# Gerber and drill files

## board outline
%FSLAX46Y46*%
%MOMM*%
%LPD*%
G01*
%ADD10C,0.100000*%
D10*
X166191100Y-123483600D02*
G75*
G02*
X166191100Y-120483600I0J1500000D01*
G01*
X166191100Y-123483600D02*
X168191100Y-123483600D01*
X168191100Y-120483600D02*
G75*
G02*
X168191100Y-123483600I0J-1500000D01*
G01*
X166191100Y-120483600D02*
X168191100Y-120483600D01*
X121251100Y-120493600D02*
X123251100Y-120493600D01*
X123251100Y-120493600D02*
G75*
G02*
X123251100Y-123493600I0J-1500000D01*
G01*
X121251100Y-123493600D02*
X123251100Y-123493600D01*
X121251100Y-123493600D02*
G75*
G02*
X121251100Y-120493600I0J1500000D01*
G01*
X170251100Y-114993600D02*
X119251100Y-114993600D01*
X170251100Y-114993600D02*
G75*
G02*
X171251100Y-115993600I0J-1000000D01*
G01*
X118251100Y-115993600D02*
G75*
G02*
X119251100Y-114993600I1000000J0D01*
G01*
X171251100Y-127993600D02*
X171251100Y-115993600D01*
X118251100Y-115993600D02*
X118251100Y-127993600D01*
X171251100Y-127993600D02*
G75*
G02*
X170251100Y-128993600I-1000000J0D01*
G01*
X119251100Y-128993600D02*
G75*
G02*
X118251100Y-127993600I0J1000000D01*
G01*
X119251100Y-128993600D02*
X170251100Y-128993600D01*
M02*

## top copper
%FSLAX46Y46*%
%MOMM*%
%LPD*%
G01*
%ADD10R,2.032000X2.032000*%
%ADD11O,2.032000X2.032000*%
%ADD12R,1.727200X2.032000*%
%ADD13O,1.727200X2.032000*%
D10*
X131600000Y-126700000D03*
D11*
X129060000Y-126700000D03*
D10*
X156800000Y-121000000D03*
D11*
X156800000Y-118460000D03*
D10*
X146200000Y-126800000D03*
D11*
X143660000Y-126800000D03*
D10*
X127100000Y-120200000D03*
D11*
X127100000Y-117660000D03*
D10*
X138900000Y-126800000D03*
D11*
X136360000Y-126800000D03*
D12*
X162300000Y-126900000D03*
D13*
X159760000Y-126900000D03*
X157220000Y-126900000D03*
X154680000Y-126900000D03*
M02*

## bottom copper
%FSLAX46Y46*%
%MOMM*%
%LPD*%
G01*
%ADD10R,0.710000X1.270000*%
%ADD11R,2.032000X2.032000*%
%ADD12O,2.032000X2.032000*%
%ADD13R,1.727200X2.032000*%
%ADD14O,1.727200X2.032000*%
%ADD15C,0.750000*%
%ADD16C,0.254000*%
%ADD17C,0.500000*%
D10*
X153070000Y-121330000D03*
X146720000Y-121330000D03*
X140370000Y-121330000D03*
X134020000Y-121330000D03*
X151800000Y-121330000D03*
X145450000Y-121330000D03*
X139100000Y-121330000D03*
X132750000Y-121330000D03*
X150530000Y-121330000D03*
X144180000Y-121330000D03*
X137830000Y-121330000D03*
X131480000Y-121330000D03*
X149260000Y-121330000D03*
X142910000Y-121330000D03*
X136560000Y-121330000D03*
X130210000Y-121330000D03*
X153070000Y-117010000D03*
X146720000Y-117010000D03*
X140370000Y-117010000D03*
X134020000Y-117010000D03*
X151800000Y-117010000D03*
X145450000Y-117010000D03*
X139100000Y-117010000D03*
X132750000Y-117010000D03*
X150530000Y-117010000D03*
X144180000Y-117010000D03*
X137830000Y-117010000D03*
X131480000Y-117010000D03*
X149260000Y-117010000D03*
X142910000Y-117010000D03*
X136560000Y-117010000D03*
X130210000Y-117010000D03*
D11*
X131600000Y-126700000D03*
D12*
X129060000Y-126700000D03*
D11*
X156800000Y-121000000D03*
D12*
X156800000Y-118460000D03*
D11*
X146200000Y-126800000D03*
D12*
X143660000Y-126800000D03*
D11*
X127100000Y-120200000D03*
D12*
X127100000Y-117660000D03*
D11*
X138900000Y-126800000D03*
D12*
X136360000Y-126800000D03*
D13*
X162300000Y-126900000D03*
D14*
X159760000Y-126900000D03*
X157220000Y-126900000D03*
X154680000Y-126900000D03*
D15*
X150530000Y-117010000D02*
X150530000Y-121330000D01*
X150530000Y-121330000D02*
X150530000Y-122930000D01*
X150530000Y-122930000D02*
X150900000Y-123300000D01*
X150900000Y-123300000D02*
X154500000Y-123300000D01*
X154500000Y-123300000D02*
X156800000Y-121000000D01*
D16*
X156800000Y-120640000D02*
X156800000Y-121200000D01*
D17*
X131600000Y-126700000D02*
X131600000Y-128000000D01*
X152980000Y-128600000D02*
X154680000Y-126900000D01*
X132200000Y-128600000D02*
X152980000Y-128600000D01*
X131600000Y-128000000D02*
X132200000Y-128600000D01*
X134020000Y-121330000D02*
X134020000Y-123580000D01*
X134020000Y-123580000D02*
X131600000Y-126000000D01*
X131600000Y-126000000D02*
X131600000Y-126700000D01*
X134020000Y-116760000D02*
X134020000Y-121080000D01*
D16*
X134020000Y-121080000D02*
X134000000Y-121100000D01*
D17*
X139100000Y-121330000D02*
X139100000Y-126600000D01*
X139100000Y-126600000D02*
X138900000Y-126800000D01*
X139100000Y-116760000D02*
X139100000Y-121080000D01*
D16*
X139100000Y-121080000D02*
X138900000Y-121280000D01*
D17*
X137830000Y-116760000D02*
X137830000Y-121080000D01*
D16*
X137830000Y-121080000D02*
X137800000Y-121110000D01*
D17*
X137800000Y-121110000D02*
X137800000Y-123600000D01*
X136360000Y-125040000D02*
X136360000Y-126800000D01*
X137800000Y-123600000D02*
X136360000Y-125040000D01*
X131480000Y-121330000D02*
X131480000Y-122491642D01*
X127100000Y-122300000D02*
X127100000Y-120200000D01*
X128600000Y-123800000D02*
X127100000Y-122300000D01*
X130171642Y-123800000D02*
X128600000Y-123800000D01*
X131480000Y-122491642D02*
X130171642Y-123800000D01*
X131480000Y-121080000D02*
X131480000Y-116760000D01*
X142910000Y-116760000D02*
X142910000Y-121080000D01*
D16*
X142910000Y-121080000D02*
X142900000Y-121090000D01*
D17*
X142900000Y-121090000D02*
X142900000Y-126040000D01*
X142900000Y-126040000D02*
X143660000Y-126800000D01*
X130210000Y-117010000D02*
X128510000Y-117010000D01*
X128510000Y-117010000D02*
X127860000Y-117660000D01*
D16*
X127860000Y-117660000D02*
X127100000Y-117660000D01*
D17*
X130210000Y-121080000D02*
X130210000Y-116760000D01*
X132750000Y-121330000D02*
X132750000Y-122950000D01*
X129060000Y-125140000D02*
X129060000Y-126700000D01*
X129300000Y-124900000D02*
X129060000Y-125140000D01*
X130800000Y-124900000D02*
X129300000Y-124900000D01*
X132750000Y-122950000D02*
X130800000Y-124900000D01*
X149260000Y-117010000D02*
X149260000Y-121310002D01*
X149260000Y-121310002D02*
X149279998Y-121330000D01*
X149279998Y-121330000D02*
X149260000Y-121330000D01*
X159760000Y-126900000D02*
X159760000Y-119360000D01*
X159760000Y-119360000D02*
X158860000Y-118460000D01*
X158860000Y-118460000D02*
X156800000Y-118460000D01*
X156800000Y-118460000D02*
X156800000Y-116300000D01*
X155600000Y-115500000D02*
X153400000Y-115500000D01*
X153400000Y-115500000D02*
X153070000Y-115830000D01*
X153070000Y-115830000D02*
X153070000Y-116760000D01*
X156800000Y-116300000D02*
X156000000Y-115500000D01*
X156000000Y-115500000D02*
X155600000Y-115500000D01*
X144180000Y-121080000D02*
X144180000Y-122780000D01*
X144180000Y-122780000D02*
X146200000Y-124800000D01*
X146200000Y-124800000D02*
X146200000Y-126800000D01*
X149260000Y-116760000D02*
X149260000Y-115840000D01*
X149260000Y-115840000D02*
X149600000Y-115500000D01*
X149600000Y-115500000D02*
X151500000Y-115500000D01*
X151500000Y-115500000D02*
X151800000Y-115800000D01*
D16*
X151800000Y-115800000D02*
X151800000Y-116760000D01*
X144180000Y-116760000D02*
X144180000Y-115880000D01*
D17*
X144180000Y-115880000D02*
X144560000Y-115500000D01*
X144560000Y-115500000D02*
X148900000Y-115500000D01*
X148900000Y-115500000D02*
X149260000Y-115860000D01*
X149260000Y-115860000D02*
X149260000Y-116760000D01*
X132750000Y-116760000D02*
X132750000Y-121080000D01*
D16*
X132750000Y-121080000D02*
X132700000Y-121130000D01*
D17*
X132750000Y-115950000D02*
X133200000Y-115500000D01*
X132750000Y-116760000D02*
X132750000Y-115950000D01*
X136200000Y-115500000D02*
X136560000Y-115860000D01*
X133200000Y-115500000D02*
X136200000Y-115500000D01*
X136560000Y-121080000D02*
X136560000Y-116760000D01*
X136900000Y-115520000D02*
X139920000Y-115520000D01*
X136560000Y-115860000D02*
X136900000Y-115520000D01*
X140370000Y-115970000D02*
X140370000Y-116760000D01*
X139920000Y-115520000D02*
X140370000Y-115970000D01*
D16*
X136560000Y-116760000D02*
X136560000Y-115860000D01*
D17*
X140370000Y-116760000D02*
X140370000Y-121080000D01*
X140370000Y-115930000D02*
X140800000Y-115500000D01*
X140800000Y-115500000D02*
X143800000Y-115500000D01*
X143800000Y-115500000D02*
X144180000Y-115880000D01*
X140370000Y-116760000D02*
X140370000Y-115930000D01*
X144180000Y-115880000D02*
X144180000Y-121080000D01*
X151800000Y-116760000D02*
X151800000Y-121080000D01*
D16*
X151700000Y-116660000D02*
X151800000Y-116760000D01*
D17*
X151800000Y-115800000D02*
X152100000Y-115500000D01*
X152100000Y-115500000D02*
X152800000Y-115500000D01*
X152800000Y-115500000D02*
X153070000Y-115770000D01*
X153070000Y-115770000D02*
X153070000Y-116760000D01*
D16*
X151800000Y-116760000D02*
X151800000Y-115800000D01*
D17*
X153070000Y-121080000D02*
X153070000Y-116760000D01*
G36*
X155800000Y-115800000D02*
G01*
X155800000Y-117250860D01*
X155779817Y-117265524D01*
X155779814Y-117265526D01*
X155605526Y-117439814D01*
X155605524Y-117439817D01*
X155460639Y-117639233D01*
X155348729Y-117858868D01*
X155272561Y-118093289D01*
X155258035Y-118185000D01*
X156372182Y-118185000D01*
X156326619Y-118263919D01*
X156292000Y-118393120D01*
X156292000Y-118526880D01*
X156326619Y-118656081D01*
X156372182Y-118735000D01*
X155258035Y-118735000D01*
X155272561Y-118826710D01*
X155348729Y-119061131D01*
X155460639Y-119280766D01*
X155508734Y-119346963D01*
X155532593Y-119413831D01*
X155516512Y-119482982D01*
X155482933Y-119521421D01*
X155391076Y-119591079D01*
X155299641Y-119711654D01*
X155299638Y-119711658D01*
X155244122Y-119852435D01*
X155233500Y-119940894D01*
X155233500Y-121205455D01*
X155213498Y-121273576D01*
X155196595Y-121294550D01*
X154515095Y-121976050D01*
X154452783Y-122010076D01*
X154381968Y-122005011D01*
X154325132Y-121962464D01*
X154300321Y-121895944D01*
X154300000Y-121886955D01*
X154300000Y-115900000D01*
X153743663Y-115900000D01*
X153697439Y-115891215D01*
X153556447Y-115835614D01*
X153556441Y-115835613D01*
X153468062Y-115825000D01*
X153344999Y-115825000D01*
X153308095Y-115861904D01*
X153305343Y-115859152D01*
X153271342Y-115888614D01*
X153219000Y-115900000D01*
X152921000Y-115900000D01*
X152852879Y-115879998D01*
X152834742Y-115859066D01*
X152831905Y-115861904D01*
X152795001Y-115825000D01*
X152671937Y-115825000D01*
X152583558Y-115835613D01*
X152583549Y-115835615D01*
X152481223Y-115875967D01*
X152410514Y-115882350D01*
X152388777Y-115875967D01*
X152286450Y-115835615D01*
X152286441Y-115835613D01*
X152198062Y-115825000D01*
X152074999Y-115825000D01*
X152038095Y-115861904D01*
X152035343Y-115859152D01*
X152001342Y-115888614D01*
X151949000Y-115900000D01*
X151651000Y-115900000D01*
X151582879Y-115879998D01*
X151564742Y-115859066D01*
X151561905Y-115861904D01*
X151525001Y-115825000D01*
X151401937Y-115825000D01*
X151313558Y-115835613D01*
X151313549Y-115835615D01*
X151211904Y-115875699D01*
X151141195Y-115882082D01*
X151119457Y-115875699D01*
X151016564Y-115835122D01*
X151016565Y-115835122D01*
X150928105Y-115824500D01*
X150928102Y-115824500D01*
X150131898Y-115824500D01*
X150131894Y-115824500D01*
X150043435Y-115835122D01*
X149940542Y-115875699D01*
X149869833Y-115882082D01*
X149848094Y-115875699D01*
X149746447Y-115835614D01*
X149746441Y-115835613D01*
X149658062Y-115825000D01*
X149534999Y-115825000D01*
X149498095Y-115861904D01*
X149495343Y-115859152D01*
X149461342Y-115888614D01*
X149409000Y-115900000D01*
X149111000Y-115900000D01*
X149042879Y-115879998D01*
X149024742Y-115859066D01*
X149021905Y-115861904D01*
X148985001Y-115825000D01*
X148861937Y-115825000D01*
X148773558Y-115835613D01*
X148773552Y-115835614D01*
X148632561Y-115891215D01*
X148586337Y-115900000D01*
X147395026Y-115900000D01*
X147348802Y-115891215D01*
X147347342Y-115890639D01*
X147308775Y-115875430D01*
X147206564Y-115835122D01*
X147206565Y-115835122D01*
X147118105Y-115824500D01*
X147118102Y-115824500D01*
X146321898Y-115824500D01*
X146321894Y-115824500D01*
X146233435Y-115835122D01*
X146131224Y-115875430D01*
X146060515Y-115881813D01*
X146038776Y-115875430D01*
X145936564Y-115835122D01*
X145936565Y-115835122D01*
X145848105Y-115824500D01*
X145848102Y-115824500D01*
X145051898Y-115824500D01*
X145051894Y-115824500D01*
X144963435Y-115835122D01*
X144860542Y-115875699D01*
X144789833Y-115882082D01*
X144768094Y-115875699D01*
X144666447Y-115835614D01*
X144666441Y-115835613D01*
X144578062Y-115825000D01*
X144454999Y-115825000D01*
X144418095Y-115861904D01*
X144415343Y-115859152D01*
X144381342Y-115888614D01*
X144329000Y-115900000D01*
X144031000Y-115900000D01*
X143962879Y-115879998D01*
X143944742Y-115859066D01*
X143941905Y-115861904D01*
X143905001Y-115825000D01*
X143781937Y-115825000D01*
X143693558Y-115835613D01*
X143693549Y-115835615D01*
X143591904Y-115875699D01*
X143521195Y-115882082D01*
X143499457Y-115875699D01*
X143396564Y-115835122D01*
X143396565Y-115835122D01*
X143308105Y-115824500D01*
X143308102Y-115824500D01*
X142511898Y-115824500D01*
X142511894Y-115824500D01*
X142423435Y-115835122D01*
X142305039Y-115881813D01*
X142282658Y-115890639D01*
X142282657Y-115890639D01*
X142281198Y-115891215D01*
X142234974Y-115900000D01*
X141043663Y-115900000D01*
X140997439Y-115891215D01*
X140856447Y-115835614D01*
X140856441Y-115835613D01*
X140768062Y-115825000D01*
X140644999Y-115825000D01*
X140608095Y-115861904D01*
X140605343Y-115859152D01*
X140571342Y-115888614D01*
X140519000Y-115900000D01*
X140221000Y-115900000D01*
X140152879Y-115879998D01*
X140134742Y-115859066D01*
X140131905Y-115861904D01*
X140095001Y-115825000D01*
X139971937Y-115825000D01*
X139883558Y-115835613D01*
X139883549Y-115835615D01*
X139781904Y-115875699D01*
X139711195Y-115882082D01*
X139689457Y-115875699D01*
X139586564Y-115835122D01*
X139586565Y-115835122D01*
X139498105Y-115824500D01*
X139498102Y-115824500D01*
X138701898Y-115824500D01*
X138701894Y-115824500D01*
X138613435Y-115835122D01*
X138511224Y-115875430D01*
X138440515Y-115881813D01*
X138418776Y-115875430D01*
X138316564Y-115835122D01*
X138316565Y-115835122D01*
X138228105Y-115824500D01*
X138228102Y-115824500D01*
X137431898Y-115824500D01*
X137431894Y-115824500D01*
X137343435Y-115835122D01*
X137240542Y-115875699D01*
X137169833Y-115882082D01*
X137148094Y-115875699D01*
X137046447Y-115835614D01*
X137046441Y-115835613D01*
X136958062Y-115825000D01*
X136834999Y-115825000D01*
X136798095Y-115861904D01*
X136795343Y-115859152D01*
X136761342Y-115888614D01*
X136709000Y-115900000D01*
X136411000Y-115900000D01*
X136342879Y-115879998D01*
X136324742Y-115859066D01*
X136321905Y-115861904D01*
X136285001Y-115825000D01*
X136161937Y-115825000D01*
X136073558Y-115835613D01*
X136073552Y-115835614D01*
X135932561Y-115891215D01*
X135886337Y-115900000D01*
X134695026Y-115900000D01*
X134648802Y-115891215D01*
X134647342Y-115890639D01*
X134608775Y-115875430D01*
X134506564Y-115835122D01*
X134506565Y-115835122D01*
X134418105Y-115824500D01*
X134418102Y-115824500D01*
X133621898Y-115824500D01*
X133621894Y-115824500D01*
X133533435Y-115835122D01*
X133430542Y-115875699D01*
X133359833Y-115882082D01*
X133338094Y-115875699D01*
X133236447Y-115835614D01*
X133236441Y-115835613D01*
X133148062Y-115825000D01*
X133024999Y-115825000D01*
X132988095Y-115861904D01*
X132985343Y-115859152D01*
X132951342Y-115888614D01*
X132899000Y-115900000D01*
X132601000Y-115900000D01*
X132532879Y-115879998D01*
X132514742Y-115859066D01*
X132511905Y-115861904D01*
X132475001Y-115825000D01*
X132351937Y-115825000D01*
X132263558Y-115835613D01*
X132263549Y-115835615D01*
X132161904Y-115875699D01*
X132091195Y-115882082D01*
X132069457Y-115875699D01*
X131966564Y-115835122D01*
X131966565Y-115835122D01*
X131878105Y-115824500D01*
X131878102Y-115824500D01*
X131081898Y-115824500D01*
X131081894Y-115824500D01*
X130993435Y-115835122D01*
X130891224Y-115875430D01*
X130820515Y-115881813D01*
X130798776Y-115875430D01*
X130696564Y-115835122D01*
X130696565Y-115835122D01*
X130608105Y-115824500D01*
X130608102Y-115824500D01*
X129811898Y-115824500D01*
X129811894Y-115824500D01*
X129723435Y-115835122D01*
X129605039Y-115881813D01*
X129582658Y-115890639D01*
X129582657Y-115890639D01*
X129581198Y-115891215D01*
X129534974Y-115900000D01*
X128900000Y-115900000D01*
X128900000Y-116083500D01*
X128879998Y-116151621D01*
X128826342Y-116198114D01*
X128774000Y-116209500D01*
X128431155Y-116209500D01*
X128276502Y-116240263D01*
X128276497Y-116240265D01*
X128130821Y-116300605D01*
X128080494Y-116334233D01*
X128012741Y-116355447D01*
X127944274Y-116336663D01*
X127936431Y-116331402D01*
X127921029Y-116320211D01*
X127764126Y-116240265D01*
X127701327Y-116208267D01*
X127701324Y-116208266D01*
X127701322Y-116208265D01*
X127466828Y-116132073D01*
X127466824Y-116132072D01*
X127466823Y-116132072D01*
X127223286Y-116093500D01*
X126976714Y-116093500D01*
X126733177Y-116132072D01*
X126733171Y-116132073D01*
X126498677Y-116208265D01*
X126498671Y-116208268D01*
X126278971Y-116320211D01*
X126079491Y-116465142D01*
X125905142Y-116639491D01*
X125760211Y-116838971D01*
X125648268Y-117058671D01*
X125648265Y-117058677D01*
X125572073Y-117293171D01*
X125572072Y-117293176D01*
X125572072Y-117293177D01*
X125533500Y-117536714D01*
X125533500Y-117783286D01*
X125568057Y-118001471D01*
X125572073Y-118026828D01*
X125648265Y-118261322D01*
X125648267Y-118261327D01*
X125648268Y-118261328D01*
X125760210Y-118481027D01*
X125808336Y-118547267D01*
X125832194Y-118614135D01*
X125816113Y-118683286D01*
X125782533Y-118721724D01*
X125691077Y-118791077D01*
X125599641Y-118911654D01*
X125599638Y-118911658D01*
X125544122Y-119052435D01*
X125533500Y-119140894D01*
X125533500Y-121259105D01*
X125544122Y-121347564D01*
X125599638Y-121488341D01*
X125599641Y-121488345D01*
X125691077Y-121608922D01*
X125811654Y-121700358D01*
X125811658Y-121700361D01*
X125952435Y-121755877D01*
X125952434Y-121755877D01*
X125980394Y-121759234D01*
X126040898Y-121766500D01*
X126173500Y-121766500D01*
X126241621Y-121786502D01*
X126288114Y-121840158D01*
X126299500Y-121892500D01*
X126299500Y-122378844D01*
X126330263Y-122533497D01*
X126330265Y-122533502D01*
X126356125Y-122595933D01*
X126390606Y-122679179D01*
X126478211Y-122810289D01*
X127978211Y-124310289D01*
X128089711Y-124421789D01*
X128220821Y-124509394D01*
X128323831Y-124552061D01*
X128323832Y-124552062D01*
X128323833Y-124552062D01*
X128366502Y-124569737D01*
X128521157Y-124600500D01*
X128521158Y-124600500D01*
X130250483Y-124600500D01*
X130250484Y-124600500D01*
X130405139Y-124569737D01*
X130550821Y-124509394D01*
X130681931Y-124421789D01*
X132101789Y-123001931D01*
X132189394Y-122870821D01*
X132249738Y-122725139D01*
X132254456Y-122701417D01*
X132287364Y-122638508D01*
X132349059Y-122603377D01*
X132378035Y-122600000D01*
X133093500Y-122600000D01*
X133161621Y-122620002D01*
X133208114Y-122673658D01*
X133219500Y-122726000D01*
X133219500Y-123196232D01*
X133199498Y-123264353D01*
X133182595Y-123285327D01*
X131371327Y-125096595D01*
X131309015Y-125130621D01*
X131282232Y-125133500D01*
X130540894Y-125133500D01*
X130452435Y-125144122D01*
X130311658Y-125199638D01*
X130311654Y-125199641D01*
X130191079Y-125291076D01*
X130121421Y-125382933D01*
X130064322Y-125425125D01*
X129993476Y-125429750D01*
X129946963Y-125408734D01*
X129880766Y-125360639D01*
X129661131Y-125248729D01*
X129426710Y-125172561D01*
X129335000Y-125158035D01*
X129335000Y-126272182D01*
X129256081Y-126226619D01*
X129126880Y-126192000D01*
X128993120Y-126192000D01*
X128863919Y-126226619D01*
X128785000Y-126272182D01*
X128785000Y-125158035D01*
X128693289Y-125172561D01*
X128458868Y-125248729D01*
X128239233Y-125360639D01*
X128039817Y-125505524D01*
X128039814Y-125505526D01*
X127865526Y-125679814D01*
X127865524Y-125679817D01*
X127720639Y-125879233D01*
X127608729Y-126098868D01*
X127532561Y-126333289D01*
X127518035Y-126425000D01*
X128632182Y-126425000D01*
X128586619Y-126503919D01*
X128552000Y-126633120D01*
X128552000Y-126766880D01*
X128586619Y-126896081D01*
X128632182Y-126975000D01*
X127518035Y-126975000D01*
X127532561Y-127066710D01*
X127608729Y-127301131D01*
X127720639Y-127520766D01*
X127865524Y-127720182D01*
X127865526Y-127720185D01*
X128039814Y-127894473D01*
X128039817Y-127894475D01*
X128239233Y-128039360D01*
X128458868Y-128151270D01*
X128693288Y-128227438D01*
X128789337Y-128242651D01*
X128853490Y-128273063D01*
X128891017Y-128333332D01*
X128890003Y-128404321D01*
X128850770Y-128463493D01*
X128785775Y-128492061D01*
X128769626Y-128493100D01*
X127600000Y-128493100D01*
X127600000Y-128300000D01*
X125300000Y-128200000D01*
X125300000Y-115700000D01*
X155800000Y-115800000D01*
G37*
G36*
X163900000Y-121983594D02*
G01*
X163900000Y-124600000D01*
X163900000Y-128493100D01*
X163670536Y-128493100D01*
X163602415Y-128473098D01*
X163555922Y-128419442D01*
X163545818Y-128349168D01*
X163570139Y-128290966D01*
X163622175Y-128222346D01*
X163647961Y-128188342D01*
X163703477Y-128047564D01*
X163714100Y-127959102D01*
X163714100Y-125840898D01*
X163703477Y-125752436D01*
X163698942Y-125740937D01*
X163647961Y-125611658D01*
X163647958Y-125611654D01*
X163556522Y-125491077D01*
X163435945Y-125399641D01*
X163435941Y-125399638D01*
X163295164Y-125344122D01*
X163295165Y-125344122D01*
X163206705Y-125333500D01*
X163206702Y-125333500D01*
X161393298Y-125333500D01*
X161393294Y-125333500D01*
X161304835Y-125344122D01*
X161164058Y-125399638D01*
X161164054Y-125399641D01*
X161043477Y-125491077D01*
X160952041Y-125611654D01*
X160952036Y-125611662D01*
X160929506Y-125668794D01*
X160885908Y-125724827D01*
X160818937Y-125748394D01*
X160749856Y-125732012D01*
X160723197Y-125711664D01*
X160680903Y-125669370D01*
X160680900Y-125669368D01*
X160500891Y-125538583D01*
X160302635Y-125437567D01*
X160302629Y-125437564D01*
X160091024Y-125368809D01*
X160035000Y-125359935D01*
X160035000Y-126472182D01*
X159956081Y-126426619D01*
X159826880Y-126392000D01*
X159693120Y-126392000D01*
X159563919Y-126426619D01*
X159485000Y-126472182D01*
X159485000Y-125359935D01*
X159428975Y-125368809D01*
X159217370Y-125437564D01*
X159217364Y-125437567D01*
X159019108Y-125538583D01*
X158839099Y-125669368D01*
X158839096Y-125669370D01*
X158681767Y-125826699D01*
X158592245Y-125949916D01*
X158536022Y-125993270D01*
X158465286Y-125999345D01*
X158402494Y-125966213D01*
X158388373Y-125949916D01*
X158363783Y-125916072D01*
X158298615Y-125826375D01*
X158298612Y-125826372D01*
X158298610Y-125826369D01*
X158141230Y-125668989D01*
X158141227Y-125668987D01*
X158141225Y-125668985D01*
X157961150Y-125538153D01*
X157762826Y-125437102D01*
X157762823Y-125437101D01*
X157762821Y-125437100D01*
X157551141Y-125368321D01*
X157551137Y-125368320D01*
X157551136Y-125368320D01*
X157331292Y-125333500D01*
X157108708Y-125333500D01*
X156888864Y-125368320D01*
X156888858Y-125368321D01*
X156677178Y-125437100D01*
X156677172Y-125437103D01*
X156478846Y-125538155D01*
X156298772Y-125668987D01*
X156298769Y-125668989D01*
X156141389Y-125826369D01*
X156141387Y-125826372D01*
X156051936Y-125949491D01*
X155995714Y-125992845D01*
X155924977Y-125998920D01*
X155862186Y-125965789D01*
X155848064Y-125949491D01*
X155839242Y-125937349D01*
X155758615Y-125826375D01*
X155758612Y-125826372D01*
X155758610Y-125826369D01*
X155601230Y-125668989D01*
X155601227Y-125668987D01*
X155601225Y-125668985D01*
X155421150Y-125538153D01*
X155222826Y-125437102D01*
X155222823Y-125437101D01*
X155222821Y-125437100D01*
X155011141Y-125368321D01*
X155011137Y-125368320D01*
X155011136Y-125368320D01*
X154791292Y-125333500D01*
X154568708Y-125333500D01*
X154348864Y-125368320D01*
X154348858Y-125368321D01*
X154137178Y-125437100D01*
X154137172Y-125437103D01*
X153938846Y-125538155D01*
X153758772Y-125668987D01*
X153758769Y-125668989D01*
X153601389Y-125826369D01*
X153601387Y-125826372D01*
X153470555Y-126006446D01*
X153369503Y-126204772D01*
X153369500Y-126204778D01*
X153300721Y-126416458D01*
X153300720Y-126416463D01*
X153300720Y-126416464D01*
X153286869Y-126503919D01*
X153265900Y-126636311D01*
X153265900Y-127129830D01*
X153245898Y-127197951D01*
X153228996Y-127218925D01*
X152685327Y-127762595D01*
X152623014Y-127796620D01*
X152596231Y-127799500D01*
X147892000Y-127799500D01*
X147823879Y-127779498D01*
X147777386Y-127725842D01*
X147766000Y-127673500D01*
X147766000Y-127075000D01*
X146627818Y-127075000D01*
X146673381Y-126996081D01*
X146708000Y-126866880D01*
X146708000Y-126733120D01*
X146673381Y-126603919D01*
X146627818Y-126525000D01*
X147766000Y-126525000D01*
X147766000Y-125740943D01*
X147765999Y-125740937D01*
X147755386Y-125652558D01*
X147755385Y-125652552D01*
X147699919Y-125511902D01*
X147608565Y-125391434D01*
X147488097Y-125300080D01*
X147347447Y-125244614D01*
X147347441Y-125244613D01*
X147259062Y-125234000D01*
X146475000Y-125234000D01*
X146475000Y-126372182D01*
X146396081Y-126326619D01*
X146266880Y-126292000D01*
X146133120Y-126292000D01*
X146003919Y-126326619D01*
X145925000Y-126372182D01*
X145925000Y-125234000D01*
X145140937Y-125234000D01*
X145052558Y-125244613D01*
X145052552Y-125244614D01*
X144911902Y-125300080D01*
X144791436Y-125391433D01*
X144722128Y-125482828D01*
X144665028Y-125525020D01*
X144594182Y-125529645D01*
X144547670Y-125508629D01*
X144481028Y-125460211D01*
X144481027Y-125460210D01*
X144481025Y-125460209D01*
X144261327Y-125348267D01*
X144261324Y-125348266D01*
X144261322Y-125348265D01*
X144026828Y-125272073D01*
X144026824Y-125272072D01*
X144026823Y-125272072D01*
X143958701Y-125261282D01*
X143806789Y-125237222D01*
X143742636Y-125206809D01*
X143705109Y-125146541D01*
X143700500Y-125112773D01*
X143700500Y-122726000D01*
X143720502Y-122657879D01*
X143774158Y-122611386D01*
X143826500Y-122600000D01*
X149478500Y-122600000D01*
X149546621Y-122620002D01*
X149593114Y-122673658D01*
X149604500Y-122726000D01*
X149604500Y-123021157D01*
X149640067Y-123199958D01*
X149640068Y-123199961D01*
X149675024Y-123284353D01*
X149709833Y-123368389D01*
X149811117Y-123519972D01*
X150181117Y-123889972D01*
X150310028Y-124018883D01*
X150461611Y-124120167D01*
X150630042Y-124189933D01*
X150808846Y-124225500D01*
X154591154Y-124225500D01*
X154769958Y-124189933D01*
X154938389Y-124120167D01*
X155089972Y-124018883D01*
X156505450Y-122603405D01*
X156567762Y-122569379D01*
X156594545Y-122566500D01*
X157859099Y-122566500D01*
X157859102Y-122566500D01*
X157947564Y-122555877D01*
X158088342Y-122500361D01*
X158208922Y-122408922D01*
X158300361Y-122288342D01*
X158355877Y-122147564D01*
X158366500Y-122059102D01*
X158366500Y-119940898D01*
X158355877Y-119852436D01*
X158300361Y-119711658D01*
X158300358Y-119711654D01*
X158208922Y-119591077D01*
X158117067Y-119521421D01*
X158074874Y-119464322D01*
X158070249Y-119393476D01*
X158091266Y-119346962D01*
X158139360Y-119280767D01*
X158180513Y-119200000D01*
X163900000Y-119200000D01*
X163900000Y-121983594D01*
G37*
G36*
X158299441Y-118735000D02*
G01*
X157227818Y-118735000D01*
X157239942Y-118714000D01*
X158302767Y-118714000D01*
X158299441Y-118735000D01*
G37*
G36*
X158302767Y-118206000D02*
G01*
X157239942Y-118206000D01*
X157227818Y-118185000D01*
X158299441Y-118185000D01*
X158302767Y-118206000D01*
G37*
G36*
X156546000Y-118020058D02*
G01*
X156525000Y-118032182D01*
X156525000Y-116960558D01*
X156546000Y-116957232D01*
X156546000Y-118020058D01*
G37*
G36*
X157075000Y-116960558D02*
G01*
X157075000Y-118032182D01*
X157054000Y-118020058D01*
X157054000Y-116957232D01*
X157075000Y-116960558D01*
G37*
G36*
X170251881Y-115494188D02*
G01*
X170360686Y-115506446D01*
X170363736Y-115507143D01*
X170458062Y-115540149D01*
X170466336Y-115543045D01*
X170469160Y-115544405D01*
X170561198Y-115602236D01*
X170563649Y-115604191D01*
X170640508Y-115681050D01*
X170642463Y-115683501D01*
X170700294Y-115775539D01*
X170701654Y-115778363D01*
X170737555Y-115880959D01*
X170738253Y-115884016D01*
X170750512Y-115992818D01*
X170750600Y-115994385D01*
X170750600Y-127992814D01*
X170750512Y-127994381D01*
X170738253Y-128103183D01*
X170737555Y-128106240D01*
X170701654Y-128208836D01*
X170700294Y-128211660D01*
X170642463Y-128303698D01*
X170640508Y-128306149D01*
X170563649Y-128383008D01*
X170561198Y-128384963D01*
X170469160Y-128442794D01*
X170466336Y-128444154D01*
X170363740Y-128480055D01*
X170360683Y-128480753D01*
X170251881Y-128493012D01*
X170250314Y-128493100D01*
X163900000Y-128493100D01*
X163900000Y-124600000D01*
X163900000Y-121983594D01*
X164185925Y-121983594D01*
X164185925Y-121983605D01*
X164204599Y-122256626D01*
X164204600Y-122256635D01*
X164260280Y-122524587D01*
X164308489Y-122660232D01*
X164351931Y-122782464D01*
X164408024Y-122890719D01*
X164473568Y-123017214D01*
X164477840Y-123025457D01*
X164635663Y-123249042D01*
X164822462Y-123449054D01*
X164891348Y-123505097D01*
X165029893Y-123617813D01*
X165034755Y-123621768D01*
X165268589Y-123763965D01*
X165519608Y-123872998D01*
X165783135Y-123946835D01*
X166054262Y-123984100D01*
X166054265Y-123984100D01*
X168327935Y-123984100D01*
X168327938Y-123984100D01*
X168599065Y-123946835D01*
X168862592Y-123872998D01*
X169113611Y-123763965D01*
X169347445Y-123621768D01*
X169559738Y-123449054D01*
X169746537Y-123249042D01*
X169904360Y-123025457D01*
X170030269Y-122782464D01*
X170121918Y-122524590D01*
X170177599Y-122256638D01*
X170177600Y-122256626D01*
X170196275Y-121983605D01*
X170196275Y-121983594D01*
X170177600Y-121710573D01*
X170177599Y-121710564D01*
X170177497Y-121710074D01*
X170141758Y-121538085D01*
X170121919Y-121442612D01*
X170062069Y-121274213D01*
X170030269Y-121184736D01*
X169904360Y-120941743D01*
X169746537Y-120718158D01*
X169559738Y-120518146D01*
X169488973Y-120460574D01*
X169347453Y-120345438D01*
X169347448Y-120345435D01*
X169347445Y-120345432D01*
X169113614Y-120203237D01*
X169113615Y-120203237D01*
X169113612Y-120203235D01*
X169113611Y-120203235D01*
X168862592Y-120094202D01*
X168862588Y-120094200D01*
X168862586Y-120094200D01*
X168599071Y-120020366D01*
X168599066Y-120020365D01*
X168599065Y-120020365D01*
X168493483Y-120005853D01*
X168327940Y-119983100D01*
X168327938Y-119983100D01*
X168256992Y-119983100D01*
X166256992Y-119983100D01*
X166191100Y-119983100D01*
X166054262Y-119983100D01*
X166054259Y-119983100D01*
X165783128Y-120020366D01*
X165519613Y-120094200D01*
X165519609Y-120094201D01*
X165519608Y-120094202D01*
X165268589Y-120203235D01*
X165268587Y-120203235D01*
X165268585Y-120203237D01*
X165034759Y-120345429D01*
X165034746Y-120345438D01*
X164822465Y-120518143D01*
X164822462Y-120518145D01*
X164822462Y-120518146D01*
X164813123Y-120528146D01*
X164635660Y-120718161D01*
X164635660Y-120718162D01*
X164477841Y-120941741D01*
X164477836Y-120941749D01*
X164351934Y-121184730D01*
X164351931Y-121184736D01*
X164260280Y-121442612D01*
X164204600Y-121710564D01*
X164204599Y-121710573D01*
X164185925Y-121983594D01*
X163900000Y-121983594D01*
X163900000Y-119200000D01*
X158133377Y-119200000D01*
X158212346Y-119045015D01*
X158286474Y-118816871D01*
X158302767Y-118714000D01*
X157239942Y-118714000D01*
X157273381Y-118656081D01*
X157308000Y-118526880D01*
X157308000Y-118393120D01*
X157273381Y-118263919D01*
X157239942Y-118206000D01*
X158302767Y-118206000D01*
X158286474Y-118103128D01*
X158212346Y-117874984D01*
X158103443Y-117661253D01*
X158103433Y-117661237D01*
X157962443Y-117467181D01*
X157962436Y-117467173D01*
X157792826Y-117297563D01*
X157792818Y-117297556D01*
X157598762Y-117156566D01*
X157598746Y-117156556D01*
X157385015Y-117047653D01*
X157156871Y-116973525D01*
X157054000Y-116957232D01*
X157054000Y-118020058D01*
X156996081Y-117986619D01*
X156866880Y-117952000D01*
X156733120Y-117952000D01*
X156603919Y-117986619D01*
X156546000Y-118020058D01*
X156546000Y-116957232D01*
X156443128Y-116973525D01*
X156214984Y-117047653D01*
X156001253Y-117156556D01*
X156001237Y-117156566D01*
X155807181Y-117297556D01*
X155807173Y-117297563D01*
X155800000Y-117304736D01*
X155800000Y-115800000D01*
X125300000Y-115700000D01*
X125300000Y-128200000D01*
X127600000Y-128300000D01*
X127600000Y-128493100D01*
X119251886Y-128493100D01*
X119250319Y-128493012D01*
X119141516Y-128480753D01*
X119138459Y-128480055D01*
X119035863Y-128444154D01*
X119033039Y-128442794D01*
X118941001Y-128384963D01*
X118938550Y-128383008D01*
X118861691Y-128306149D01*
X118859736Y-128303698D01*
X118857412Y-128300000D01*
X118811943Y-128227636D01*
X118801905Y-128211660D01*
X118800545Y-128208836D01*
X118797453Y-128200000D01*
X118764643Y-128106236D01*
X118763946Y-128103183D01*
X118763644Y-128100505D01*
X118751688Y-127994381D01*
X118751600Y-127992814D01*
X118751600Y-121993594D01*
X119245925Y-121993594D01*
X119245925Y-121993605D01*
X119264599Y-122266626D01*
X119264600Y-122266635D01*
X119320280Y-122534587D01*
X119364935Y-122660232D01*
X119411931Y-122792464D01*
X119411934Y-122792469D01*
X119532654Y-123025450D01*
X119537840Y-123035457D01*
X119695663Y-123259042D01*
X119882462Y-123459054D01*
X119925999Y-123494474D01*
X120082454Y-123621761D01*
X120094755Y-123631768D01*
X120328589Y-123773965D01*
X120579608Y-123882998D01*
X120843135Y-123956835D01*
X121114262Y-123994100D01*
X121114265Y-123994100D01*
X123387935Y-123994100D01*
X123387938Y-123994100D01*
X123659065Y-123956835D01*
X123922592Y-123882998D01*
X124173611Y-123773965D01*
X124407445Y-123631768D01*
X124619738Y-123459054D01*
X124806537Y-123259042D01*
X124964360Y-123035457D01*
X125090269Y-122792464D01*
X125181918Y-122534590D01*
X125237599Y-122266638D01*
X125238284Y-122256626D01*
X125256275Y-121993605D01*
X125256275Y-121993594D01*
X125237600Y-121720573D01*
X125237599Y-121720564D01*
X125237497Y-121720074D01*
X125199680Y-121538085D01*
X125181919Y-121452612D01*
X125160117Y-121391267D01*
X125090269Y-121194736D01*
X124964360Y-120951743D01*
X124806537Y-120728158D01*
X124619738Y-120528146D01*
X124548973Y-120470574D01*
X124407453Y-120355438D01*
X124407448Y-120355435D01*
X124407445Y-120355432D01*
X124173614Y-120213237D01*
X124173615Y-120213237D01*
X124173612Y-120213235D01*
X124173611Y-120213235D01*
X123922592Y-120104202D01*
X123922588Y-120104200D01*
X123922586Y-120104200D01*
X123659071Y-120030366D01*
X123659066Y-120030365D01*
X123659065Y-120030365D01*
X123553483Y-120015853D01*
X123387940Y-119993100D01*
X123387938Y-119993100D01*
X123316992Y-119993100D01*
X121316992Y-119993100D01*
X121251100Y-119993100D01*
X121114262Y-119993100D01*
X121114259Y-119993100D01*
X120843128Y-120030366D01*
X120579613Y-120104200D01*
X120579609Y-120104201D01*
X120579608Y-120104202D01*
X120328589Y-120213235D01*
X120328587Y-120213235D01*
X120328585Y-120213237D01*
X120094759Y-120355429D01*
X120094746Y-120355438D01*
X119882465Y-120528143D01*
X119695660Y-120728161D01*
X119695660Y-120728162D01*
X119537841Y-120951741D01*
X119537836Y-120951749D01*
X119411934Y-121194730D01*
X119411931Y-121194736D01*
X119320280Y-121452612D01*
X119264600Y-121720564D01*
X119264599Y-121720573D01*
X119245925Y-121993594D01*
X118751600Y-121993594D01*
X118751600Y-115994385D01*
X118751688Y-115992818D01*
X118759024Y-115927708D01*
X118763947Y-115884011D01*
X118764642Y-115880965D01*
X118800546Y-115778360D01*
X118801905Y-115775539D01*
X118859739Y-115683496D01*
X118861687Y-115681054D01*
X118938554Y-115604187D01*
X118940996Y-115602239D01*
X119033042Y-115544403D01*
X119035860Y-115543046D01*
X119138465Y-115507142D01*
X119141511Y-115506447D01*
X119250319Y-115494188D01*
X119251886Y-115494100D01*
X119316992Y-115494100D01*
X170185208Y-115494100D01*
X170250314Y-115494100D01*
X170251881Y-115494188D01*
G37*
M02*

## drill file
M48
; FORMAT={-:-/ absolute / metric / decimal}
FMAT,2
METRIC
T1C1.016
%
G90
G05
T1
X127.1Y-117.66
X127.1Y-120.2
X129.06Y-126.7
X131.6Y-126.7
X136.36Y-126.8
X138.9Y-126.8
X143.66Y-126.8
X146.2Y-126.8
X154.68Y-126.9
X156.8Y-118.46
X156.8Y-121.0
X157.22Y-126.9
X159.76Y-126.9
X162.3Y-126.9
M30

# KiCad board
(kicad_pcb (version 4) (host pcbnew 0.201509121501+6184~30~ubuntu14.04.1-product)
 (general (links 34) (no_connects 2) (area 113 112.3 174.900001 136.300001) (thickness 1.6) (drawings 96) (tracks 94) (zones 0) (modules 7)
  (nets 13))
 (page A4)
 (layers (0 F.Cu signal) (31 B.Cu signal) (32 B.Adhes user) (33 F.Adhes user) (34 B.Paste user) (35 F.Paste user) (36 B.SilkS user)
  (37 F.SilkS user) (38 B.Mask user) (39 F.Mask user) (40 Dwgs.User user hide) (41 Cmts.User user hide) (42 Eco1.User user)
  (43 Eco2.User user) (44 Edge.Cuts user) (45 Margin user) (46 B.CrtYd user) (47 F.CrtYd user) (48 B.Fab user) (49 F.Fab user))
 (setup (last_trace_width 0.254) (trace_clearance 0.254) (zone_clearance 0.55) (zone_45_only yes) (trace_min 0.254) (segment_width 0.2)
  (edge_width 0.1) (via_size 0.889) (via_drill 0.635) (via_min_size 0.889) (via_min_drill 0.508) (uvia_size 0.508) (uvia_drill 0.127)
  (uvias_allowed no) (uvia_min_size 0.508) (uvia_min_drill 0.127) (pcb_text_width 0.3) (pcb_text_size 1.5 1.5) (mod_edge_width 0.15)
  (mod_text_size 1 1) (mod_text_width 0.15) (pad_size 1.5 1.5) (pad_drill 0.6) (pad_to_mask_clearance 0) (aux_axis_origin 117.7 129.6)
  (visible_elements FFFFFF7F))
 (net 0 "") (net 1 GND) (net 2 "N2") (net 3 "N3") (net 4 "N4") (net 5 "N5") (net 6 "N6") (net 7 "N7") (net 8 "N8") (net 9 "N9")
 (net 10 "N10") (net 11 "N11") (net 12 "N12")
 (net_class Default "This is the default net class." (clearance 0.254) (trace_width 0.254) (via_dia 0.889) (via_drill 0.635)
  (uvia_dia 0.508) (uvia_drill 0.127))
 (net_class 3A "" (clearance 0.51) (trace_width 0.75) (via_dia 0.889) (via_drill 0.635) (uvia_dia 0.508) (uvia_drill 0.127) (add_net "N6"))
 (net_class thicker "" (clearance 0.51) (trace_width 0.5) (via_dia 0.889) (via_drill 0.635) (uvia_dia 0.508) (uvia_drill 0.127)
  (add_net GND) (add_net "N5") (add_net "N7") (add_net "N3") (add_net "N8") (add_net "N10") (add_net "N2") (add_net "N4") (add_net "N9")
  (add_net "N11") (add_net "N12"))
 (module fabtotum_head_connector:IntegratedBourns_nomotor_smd (layer B.Cu) (at 153 121.35 90)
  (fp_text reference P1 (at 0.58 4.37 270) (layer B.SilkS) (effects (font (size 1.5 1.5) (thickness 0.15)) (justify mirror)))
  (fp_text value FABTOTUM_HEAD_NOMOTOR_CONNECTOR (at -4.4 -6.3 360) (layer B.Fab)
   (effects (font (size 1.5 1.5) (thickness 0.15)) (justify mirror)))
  (pad 1 smd rect (at 0.02 0.07 90) (size 1.27 0.71) (layers B.Cu B.Paste B.Mask) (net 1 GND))
  (pad 5 smd rect (at 0.02 -6.28 90) (size 1.27 0.71) (layers B.Cu B.Paste B.Mask) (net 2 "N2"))
  (pad 9 smd rect (at 0.02 -12.63 90) (size 1.27 0.71) (layers B.Cu B.Paste B.Mask) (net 1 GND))
  (pad 13 smd rect (at 0.02 -18.98 90) (size 1.27 0.71) (layers B.Cu B.Paste B.Mask) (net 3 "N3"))
  (pad 2 smd rect (at 0.02 -1.2 90) (size 1.27 0.71) (layers B.Cu B.Paste B.Mask) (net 1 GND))
  (pad 6 smd rect (at 0.02 -7.55 90) (size 1.27 0.71) (layers B.Cu B.Paste B.Mask) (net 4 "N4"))
  (pad 10 smd rect (at 0.02 -13.9 90) (size 1.27 0.71) (layers B.Cu B.Paste B.Mask) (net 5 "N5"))
  (pad 14 smd rect (at 0.02 -20.25 90) (size 1.27 0.71) (layers B.Cu B.Paste B.Mask) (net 1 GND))
  (pad 3 smd rect (at 0.02 -2.47 90) (size 1.27 0.71) (layers B.Cu B.Paste B.Mask) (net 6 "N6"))
  (pad 7 smd rect (at 0.02 -8.82 90) (size 1.27 0.71) (layers B.Cu B.Paste B.Mask) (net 1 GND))
  (pad 11 smd rect (at 0.02 -15.17 90) (size 1.27 0.71) (layers B.Cu B.Paste B.Mask) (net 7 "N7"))
  (pad 15 smd rect (at 0.02 -21.52 90) (size 1.27 0.71) (layers B.Cu B.Paste B.Mask) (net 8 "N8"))
  (pad 4 smd rect (at 0.02 -3.74 90) (size 1.27 0.71) (layers B.Cu B.Paste B.Mask) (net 1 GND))
  (pad 8 smd rect (at 0.02 -10.09 90) (size 1.27 0.71) (layers B.Cu B.Paste B.Mask) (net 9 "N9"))
  (pad 12 smd rect (at 0.02 -16.44 90) (size 1.27 0.71) (layers B.Cu B.Paste B.Mask) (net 1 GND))
  (pad 16 smd rect (at 0.02 -22.79 90) (size 1.27 0.71) (layers B.Cu B.Paste B.Mask) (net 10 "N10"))
  (pad 1 smd rect (at 4.34 0.07 90) (size 1.27 0.71) (layers B.Cu B.Paste B.Mask) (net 1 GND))
  (pad 5 smd rect (at 4.34 -6.28 90) (size 1.27 0.71) (layers B.Cu B.Paste B.Mask) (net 2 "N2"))
  (pad 9 smd rect (at 4.34 -12.63 90) (size 1.27 0.71) (layers B.Cu B.Paste B.Mask) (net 1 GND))
  (pad 13 smd rect (at 4.34 -18.98 90) (size 1.27 0.71) (layers B.Cu B.Paste B.Mask) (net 3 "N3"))
  (pad 2 smd rect (at 4.34 -1.2 90) (size 1.27 0.71) (layers B.Cu B.Paste B.Mask) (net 1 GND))
  (pad 6 smd rect (at 4.34 -7.55 90) (size 1.27 0.71) (layers B.Cu B.Paste B.Mask) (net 4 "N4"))
  (pad 10 smd rect (at 4.34 -13.9 90) (size 1.27 0.71) (layers B.Cu B.Paste B.Mask) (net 5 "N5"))
  (pad 14 smd rect (at 4.34 -20.25 90) (size 1.27 0.71) (layers B.Cu B.Paste B.Mask) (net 1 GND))
  (pad 3 smd rect (at 4.34 -2.47 90) (size 1.27 0.71) (layers B.Cu B.Paste B.Mask) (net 6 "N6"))
  (pad 7 smd rect (at 4.34 -8.82 90) (size 1.27 0.71) (layers B.Cu B.Paste B.Mask) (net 1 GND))
  (pad 11 smd rect (at 4.34 -15.17 90) (size 1.27 0.71) (layers B.Cu B.Paste B.Mask) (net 7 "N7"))
  (pad 15 smd rect (at 4.34 -21.52 90) (size 1.27 0.71) (layers B.Cu B.Paste B.Mask) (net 8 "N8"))
  (pad 4 smd rect (at 4.34 -3.74 90) (size 1.27 0.71) (layers B.Cu B.Paste B.Mask) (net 1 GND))
  (pad 8 smd rect (at 4.34 -10.09 90) (size 1.27 0.71) (layers B.Cu B.Paste B.Mask) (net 9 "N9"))
  (pad 12 smd rect (at 4.34 -16.44 90) (size 1.27 0.71) (layers B.Cu B.Paste B.Mask) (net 1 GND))
  (pad 16 smd rect (at 4.34 -22.79 90) (size 1.27 0.71) (layers B.Cu B.Paste B.Mask) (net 10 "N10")))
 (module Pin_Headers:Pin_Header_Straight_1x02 (layer F.Cu) (at 131.6 126.7 270)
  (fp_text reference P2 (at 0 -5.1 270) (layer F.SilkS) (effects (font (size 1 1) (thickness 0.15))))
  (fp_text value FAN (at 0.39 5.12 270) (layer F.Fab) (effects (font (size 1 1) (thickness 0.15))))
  (pad 1 thru_hole rect (at 0 0 270) (size 2.032 2.032) (drill 1.016) (layers *.Cu *.Mask F.SilkS) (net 3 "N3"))
  (pad 2 thru_hole oval (at 0 2.54 270) (size 2.032 2.032) (drill 1.016) (layers *.Cu *.Mask F.SilkS) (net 1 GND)))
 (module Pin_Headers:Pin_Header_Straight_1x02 (layer F.Cu) (at 156.8 121 180)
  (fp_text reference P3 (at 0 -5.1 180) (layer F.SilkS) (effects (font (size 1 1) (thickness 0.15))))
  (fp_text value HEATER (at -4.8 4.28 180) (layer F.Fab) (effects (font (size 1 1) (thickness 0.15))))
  (pad 1 thru_hole rect (at 0 0 180) (size 2.032 2.032) (drill 1.016) (layers *.Cu *.Mask F.SilkS) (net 6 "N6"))
  (pad 2 thru_hole oval (at 0 2.54 180) (size 2.032 2.032) (drill 1.016) (layers *.Cu *.Mask F.SilkS) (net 1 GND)))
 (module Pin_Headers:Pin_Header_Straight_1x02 (layer F.Cu) (at 146.2 126.8 270)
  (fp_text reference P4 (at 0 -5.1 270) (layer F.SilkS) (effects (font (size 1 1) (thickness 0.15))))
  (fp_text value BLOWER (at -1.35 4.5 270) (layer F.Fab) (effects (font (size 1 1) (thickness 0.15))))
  (pad 1 thru_hole rect (at 0 0 270) (size 2.032 2.032) (drill 1.016) (layers *.Cu *.Mask F.SilkS) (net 1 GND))
  (pad 2 thru_hole oval (at 0 2.54 270) (size 2.032 2.032) (drill 1.016) (layers *.Cu *.Mask F.SilkS) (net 9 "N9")))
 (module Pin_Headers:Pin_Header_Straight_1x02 (layer F.Cu) (at 127.1 120.2 180)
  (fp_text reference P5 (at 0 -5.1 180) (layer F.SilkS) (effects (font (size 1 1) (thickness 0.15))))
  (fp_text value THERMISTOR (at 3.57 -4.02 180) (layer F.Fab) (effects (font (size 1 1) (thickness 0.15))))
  (pad 1 thru_hole rect (at 0 0 180) (size 2.032 2.032) (drill 1.016) (layers *.Cu *.Mask F.SilkS) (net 8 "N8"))
  (pad 2 thru_hole oval (at 0 2.54 180) (size 2.032 2.032) (drill 1.016) (layers *.Cu *.Mask F.SilkS) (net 10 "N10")))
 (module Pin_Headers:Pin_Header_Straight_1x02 (layer F.Cu) (at 138.9 126.8 270)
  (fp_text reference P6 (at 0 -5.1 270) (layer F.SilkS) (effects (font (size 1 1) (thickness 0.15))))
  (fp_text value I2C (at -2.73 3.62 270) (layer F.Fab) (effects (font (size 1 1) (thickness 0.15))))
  (pad 1 thru_hole rect (at 0 0 270) (size 2.032 2.032) (drill 1.016) (layers *.Cu *.Mask F.SilkS) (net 5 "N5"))
  (pad 2 thru_hole oval (at 0 2.54 270) (size 2.032 2.032) (drill 1.016) (layers *.Cu *.Mask F.SilkS) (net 7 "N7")))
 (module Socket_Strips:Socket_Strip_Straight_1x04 (layer F.Cu) (at 162.3 126.9 180)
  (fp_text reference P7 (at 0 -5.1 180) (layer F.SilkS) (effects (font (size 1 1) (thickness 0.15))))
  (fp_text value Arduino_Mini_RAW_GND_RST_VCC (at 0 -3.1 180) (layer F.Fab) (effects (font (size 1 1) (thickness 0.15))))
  (pad 1 thru_hole rect (at 0 0 180) (size 1.7272 2.032) (drill 1.016) (layers *.Cu *.Mask F.SilkS) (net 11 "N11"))
  (pad 2 thru_hole oval (at 2.54 0 180) (size 1.7272 2.032) (drill 1.016) (layers *.Cu *.Mask F.SilkS) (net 1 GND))
  (pad 3 thru_hole oval (at 5.08 0 180) (size 1.7272 2.032) (drill 1.016) (layers *.Cu *.Mask F.SilkS) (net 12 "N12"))
  (pad 4 thru_hole oval (at 7.62 0 180) (size 1.7272 2.032) (drill 1.016) (layers *.Cu *.Mask F.SilkS) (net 3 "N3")))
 (gr_arc (start 166.1911 121.9836) (end 166.1911 120.4836) (angle -180) (layer Edge.Cuts) (width 0.1))
 (gr_line (start 166.1911 123.4836) (end 168.1911 123.4836) (layer Edge.Cuts) (width 0.1))
 (gr_arc (start 168.1911 121.9836) (end 168.1911 123.4836) (angle -180) (layer Edge.Cuts) (width 0.1))
 (gr_line (start 166.1911 120.4836) (end 168.1911 120.4836) (layer Edge.Cuts) (width 0.1))
 (gr_line (start 121.2511 120.4936) (end 123.2511 120.4936) (layer Edge.Cuts) (width 0.1))
 (gr_arc (start 123.2511 121.9936) (end 123.2511 123.4936) (angle -180) (layer Edge.Cuts) (width 0.1))
 (gr_line (start 121.2511 123.4936) (end 123.2511 123.4936) (layer Edge.Cuts) (width 0.1))
 (gr_arc (start 121.2511 121.9936) (end 121.2511 120.4936) (angle -180) (layer Edge.Cuts) (width 0.1))
 (gr_line (start 170.2511 114.9936) (end 119.2511 114.9936) (layer Edge.Cuts) (width 0.1))
 (gr_arc (start 170.2511 115.9936) (end 171.2511 115.9936) (angle -90) (layer Edge.Cuts) (width 0.1))
 (gr_arc (start 119.2511 115.9936) (end 119.2511 114.9936) (angle -90) (layer Edge.Cuts) (width 0.1))
 (gr_line (start 171.2511 127.9936) (end 171.2511 115.9936) (layer Edge.Cuts) (width 0.1))
 (gr_line (start 118.2511 115.9936) (end 118.2511 127.9936) (layer Edge.Cuts) (width 0.1))
 (gr_arc (start 170.2511 127.9936) (end 170.2511 128.9936) (angle -90) (layer Edge.Cuts) (width 0.1))
 (gr_arc (start 119.2511 127.9936) (end 118.2511 127.9936) (angle -90) (layer Edge.Cuts) (width 0.1))
 (gr_line (start 119.2511 128.9936) (end 170.2511 128.9936) (layer Edge.Cuts) (width 0.1))
 (segment (start 150.53 117.01) (end 150.53 121.33) (width 0.75) (layer B.Cu) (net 6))
 (segment (start 150.53 121.33) (end 150.53 122.93) (width 0.75) (layer B.Cu) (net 6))
 (segment (start 150.53 122.93) (end 150.9 123.3) (width 0.75) (layer B.Cu) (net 6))
 (segment (start 150.9 123.3) (end 154.5 123.3) (width 0.75) (layer B.Cu) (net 6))
 (segment (start 154.5 123.3) (end 156.8 121) (width 0.75) (layer B.Cu) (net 6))
 (segment (start 156.8 120.64) (end 156.8 121.2) (width 0.254) (layer B.Cu) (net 6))
 (segment (start 131.6 126.7) (end 131.6 128) (width 0.5) (layer B.Cu) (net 3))
 (segment (start 152.98 128.6) (end 154.68 126.9) (width 0.5) (layer B.Cu) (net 3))
 (segment (start 132.2 128.6) (end 152.98 128.6) (width 0.5) (layer B.Cu) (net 3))
 (segment (start 131.6 128) (end 132.2 128.6) (width 0.5) (layer B.Cu) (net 3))
 (segment (start 134.02 121.33) (end 134.02 123.58) (width 0.5) (layer B.Cu) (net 3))
 (segment (start 134.02 123.58) (end 131.6 126) (width 0.5) (layer B.Cu) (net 3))
 (segment (start 131.6 126) (end 131.6 126.7) (width 0.5) (layer B.Cu) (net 3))
 (segment (start 134.02 116.76) (end 134.02 121.08) (width 0.5) (layer B.Cu) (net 3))
 (segment (start 134.02 121.08) (end 134 121.1) (width 0.254) (layer B.Cu) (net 3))
 (segment (start 139.1 121.33) (end 139.1 126.6) (width 0.5) (layer B.Cu) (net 5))
 (segment (start 139.1 126.6) (end 138.9 126.8) (width 0.5) (layer B.Cu) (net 5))
 (segment (start 139.1 116.76) (end 139.1 121.08) (width 0.5) (layer B.Cu) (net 5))
 (segment (start 139.1 121.08) (end 138.9 121.28) (width 0.254) (layer B.Cu) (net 5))
 (segment (start 137.83 116.76) (end 137.83 121.08) (width 0.5) (layer B.Cu) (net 7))
 (segment (start 137.83 121.08) (end 137.8 121.11) (width 0.254) (layer B.Cu) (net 7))
 (segment (start 137.8 121.11) (end 137.8 123.6) (width 0.5) (layer B.Cu) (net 7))
 (segment (start 136.36 125.04) (end 136.36 126.8) (width 0.5) (layer B.Cu) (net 7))
 (segment (start 137.8 123.6) (end 136.36 125.04) (width 0.5) (layer B.Cu) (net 7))
 (segment (start 131.48 121.33) (end 131.48 122.491642) (width 0.5) (layer B.Cu) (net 8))
 (segment (start 127.1 122.3) (end 127.1 120.2) (width 0.5) (layer B.Cu) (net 8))
 (segment (start 128.6 123.8) (end 127.1 122.3) (width 0.5) (layer B.Cu) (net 8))
 (segment (start 130.171642 123.8) (end 128.6 123.8) (width 0.5) (layer B.Cu) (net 8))
 (segment (start 131.48 122.491642) (end 130.171642 123.8) (width 0.5) (layer B.Cu) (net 8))
 (segment (start 131.48 121.08) (end 131.48 116.76) (width 0.5) (layer B.Cu) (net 8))
 (segment (start 142.91 116.76) (end 142.91 121.08) (width 0.5) (layer B.Cu) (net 9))
 (segment (start 142.91 121.08) (end 142.9 121.09) (width 0.254) (layer B.Cu) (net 9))
 (segment (start 142.9 121.09) (end 142.9 126.04) (width 0.5) (layer B.Cu) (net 9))
 (segment (start 142.9 126.04) (end 143.66 126.8) (width 0.5) (layer B.Cu) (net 9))
 (segment (start 130.21 117.01) (end 128.51 117.01) (width 0.5) (layer B.Cu) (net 10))
 (segment (start 128.51 117.01) (end 127.86 117.66) (width 0.5) (layer B.Cu) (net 10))
 (segment (start 127.86 117.66) (end 127.1 117.66) (width 0.254) (layer B.Cu) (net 10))
 (segment (start 130.21 121.08) (end 130.21 116.76) (width 0.5) (layer B.Cu) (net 10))
 (segment (start 132.75 121.33) (end 132.75 122.95) (width 0.5) (layer B.Cu) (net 1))
 (segment (start 129.06 125.14) (end 129.06 126.7) (width 0.5) (layer B.Cu) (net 1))
 (segment (start 129.3 124.9) (end 129.06 125.14) (width 0.5) (layer B.Cu) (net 1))
 (segment (start 130.8 124.9) (end 129.3 124.9) (width 0.5) (layer B.Cu) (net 1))
 (segment (start 132.75 122.95) (end 130.8 124.9) (width 0.5) (layer B.Cu) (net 1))
 (segment (start 149.26 117.01) (end 149.26 121.310002) (width 0.5) (layer B.Cu) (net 1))
 (segment (start 149.26 121.310002) (end 149.279998 121.33) (width 0.5) (layer B.Cu) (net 1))
 (segment (start 149.279998 121.33) (end 149.26 121.33) (width 0.5) (layer B.Cu) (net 1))
 (segment (start 159.76 126.9) (end 159.76 119.36) (width 0.5) (layer B.Cu) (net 1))
 (segment (start 159.76 119.36) (end 158.86 118.46) (width 0.5) (layer B.Cu) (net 1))
 (segment (start 158.86 118.46) (end 156.8 118.46) (width 0.5) (layer B.Cu) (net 1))
 (segment (start 156.8 118.46) (end 156.8 116.3) (width 0.5) (layer B.Cu) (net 1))
 (segment (start 155.6 115.5) (end 153.4 115.5) (width 0.5) (layer B.Cu) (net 1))
 (segment (start 153.4 115.5) (end 153.07 115.83) (width 0.5) (layer B.Cu) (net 1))
 (segment (start 153.07 115.83) (end 153.07 116.76) (width 0.5) (layer B.Cu) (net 1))
 (segment (start 156.8 116.3) (end 156 115.5) (width 0.5) (layer B.Cu) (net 1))
 (segment (start 156 115.5) (end 155.6 115.5) (width 0.5) (layer B.Cu) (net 1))
 (segment (start 144.18 121.08) (end 144.18 122.78) (width 0.5) (layer B.Cu) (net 1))
 (segment (start 144.18 122.78) (end 146.2 124.8) (width 0.5) (layer B.Cu) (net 1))
 (segment (start 146.2 124.8) (end 146.2 126.8) (width 0.5) (layer B.Cu) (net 1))
 (segment (start 149.26 116.76) (end 149.26 115.84) (width 0.5) (layer B.Cu) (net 1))
 (segment (start 149.26 115.84) (end 149.6 115.5) (width 0.5) (layer B.Cu) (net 1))
 (segment (start 149.6 115.5) (end 151.5 115.5) (width 0.5) (layer B.Cu) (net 1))
 (segment (start 151.5 115.5) (end 151.8 115.8) (width 0.5) (layer B.Cu) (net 1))
 (segment (start 151.8 115.8) (end 151.8 116.76) (width 0.254) (layer B.Cu) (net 1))
 (segment (start 144.18 116.76) (end 144.18 115.88) (width 0.254) (layer B.Cu) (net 1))
 (segment (start 144.18 115.88) (end 144.56 115.5) (width 0.5) (layer B.Cu) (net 1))
 (segment (start 144.56 115.5) (end 148.9 115.5) (width 0.5) (layer B.Cu) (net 1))
 (segment (start 148.9 115.5) (end 149.26 115.86) (width 0.5) (layer B.Cu) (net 1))
 (segment (start 149.26 115.86) (end 149.26 116.76) (width 0.5) (layer B.Cu) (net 1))
 (segment (start 132.75 116.76) (end 132.75 121.08) (width 0.5) (layer B.Cu) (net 1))
 (segment (start 132.75 121.08) (end 132.7 121.13) (width 0.254) (layer B.Cu) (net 1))
 (segment (start 132.75 115.95) (end 133.2 115.5) (width 0.5) (layer B.Cu) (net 1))
 (segment (start 132.75 116.76) (end 132.75 115.95) (width 0.5) (layer B.Cu) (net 1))
 (segment (start 136.2 115.5) (end 136.56 115.86) (width 0.5) (layer B.Cu) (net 1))
 (segment (start 133.2 115.5) (end 136.2 115.5) (width 0.5) (layer B.Cu) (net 1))
 (segment (start 136.56 121.08) (end 136.56 116.76) (width 0.5) (layer B.Cu) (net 1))
 (segment (start 136.9 115.52) (end 139.92 115.52) (width 0.5) (layer B.Cu) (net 1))
 (segment (start 136.56 115.86) (end 136.9 115.52) (width 0.5) (layer B.Cu) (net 1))
 (segment (start 140.37 115.97) (end 140.37 116.76) (width 0.5) (layer B.Cu) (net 1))
 (segment (start 139.92 115.52) (end 140.37 115.97) (width 0.5) (layer B.Cu) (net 1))
 (segment (start 136.56 116.76) (end 136.56 115.86) (width 0.254) (layer B.Cu) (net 1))
 (segment (start 140.37 116.76) (end 140.37 121.08) (width 0.5) (layer B.Cu) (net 1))
 (segment (start 140.37 115.93) (end 140.8 115.5) (width 0.5) (layer B.Cu) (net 1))
 (segment (start 140.8 115.5) (end 143.8 115.5) (width 0.5) (layer B.Cu) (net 1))
 (segment (start 143.8 115.5) (end 144.18 115.88) (width 0.5) (layer B.Cu) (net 1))
 (segment (start 140.37 116.76) (end 140.37 115.93) (width 0.5) (layer B.Cu) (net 1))
 (segment (start 144.18 115.88) (end 144.18 121.08) (width 0.5) (layer B.Cu) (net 1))
 (segment (start 151.8 116.76) (end 151.8 121.08) (width 0.5) (layer B.Cu) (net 1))
 (segment (start 151.7 116.66) (end 151.8 116.76) (width 0.254) (layer B.Cu) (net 1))
 (segment (start 151.8 115.8) (end 152.1 115.5) (width 0.5) (layer B.Cu) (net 1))
 (segment (start 152.1 115.5) (end 152.8 115.5) (width 0.5) (layer B.Cu) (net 1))
 (segment (start 152.8 115.5) (end 153.07 115.77) (width 0.5) (layer B.Cu) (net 1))
 (segment (start 153.07 115.77) (end 153.07 116.76) (width 0.5) (layer B.Cu) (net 1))
 (segment (start 151.8 116.76) (end 151.8 115.8) (width 0.254) (layer B.Cu) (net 1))
 (segment (start 153.07 121.08) (end 153.07 116.76) (width 0.5) (layer B.Cu) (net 1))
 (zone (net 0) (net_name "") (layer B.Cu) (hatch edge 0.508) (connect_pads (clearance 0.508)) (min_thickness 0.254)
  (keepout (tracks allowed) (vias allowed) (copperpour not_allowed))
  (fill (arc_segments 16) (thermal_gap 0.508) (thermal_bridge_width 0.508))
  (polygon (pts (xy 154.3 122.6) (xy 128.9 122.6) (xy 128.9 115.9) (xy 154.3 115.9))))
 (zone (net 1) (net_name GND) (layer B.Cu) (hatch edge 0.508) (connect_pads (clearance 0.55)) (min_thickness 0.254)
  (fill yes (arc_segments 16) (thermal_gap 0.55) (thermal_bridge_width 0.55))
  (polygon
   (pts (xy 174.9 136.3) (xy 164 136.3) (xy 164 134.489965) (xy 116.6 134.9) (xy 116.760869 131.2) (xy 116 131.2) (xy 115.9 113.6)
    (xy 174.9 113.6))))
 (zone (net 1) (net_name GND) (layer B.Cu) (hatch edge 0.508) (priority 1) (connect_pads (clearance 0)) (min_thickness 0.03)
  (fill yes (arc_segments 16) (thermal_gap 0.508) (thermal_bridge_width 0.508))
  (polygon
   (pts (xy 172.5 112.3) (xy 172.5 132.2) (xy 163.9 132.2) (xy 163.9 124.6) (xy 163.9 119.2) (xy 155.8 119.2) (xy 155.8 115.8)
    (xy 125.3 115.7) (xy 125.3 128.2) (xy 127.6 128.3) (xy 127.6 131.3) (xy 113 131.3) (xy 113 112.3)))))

